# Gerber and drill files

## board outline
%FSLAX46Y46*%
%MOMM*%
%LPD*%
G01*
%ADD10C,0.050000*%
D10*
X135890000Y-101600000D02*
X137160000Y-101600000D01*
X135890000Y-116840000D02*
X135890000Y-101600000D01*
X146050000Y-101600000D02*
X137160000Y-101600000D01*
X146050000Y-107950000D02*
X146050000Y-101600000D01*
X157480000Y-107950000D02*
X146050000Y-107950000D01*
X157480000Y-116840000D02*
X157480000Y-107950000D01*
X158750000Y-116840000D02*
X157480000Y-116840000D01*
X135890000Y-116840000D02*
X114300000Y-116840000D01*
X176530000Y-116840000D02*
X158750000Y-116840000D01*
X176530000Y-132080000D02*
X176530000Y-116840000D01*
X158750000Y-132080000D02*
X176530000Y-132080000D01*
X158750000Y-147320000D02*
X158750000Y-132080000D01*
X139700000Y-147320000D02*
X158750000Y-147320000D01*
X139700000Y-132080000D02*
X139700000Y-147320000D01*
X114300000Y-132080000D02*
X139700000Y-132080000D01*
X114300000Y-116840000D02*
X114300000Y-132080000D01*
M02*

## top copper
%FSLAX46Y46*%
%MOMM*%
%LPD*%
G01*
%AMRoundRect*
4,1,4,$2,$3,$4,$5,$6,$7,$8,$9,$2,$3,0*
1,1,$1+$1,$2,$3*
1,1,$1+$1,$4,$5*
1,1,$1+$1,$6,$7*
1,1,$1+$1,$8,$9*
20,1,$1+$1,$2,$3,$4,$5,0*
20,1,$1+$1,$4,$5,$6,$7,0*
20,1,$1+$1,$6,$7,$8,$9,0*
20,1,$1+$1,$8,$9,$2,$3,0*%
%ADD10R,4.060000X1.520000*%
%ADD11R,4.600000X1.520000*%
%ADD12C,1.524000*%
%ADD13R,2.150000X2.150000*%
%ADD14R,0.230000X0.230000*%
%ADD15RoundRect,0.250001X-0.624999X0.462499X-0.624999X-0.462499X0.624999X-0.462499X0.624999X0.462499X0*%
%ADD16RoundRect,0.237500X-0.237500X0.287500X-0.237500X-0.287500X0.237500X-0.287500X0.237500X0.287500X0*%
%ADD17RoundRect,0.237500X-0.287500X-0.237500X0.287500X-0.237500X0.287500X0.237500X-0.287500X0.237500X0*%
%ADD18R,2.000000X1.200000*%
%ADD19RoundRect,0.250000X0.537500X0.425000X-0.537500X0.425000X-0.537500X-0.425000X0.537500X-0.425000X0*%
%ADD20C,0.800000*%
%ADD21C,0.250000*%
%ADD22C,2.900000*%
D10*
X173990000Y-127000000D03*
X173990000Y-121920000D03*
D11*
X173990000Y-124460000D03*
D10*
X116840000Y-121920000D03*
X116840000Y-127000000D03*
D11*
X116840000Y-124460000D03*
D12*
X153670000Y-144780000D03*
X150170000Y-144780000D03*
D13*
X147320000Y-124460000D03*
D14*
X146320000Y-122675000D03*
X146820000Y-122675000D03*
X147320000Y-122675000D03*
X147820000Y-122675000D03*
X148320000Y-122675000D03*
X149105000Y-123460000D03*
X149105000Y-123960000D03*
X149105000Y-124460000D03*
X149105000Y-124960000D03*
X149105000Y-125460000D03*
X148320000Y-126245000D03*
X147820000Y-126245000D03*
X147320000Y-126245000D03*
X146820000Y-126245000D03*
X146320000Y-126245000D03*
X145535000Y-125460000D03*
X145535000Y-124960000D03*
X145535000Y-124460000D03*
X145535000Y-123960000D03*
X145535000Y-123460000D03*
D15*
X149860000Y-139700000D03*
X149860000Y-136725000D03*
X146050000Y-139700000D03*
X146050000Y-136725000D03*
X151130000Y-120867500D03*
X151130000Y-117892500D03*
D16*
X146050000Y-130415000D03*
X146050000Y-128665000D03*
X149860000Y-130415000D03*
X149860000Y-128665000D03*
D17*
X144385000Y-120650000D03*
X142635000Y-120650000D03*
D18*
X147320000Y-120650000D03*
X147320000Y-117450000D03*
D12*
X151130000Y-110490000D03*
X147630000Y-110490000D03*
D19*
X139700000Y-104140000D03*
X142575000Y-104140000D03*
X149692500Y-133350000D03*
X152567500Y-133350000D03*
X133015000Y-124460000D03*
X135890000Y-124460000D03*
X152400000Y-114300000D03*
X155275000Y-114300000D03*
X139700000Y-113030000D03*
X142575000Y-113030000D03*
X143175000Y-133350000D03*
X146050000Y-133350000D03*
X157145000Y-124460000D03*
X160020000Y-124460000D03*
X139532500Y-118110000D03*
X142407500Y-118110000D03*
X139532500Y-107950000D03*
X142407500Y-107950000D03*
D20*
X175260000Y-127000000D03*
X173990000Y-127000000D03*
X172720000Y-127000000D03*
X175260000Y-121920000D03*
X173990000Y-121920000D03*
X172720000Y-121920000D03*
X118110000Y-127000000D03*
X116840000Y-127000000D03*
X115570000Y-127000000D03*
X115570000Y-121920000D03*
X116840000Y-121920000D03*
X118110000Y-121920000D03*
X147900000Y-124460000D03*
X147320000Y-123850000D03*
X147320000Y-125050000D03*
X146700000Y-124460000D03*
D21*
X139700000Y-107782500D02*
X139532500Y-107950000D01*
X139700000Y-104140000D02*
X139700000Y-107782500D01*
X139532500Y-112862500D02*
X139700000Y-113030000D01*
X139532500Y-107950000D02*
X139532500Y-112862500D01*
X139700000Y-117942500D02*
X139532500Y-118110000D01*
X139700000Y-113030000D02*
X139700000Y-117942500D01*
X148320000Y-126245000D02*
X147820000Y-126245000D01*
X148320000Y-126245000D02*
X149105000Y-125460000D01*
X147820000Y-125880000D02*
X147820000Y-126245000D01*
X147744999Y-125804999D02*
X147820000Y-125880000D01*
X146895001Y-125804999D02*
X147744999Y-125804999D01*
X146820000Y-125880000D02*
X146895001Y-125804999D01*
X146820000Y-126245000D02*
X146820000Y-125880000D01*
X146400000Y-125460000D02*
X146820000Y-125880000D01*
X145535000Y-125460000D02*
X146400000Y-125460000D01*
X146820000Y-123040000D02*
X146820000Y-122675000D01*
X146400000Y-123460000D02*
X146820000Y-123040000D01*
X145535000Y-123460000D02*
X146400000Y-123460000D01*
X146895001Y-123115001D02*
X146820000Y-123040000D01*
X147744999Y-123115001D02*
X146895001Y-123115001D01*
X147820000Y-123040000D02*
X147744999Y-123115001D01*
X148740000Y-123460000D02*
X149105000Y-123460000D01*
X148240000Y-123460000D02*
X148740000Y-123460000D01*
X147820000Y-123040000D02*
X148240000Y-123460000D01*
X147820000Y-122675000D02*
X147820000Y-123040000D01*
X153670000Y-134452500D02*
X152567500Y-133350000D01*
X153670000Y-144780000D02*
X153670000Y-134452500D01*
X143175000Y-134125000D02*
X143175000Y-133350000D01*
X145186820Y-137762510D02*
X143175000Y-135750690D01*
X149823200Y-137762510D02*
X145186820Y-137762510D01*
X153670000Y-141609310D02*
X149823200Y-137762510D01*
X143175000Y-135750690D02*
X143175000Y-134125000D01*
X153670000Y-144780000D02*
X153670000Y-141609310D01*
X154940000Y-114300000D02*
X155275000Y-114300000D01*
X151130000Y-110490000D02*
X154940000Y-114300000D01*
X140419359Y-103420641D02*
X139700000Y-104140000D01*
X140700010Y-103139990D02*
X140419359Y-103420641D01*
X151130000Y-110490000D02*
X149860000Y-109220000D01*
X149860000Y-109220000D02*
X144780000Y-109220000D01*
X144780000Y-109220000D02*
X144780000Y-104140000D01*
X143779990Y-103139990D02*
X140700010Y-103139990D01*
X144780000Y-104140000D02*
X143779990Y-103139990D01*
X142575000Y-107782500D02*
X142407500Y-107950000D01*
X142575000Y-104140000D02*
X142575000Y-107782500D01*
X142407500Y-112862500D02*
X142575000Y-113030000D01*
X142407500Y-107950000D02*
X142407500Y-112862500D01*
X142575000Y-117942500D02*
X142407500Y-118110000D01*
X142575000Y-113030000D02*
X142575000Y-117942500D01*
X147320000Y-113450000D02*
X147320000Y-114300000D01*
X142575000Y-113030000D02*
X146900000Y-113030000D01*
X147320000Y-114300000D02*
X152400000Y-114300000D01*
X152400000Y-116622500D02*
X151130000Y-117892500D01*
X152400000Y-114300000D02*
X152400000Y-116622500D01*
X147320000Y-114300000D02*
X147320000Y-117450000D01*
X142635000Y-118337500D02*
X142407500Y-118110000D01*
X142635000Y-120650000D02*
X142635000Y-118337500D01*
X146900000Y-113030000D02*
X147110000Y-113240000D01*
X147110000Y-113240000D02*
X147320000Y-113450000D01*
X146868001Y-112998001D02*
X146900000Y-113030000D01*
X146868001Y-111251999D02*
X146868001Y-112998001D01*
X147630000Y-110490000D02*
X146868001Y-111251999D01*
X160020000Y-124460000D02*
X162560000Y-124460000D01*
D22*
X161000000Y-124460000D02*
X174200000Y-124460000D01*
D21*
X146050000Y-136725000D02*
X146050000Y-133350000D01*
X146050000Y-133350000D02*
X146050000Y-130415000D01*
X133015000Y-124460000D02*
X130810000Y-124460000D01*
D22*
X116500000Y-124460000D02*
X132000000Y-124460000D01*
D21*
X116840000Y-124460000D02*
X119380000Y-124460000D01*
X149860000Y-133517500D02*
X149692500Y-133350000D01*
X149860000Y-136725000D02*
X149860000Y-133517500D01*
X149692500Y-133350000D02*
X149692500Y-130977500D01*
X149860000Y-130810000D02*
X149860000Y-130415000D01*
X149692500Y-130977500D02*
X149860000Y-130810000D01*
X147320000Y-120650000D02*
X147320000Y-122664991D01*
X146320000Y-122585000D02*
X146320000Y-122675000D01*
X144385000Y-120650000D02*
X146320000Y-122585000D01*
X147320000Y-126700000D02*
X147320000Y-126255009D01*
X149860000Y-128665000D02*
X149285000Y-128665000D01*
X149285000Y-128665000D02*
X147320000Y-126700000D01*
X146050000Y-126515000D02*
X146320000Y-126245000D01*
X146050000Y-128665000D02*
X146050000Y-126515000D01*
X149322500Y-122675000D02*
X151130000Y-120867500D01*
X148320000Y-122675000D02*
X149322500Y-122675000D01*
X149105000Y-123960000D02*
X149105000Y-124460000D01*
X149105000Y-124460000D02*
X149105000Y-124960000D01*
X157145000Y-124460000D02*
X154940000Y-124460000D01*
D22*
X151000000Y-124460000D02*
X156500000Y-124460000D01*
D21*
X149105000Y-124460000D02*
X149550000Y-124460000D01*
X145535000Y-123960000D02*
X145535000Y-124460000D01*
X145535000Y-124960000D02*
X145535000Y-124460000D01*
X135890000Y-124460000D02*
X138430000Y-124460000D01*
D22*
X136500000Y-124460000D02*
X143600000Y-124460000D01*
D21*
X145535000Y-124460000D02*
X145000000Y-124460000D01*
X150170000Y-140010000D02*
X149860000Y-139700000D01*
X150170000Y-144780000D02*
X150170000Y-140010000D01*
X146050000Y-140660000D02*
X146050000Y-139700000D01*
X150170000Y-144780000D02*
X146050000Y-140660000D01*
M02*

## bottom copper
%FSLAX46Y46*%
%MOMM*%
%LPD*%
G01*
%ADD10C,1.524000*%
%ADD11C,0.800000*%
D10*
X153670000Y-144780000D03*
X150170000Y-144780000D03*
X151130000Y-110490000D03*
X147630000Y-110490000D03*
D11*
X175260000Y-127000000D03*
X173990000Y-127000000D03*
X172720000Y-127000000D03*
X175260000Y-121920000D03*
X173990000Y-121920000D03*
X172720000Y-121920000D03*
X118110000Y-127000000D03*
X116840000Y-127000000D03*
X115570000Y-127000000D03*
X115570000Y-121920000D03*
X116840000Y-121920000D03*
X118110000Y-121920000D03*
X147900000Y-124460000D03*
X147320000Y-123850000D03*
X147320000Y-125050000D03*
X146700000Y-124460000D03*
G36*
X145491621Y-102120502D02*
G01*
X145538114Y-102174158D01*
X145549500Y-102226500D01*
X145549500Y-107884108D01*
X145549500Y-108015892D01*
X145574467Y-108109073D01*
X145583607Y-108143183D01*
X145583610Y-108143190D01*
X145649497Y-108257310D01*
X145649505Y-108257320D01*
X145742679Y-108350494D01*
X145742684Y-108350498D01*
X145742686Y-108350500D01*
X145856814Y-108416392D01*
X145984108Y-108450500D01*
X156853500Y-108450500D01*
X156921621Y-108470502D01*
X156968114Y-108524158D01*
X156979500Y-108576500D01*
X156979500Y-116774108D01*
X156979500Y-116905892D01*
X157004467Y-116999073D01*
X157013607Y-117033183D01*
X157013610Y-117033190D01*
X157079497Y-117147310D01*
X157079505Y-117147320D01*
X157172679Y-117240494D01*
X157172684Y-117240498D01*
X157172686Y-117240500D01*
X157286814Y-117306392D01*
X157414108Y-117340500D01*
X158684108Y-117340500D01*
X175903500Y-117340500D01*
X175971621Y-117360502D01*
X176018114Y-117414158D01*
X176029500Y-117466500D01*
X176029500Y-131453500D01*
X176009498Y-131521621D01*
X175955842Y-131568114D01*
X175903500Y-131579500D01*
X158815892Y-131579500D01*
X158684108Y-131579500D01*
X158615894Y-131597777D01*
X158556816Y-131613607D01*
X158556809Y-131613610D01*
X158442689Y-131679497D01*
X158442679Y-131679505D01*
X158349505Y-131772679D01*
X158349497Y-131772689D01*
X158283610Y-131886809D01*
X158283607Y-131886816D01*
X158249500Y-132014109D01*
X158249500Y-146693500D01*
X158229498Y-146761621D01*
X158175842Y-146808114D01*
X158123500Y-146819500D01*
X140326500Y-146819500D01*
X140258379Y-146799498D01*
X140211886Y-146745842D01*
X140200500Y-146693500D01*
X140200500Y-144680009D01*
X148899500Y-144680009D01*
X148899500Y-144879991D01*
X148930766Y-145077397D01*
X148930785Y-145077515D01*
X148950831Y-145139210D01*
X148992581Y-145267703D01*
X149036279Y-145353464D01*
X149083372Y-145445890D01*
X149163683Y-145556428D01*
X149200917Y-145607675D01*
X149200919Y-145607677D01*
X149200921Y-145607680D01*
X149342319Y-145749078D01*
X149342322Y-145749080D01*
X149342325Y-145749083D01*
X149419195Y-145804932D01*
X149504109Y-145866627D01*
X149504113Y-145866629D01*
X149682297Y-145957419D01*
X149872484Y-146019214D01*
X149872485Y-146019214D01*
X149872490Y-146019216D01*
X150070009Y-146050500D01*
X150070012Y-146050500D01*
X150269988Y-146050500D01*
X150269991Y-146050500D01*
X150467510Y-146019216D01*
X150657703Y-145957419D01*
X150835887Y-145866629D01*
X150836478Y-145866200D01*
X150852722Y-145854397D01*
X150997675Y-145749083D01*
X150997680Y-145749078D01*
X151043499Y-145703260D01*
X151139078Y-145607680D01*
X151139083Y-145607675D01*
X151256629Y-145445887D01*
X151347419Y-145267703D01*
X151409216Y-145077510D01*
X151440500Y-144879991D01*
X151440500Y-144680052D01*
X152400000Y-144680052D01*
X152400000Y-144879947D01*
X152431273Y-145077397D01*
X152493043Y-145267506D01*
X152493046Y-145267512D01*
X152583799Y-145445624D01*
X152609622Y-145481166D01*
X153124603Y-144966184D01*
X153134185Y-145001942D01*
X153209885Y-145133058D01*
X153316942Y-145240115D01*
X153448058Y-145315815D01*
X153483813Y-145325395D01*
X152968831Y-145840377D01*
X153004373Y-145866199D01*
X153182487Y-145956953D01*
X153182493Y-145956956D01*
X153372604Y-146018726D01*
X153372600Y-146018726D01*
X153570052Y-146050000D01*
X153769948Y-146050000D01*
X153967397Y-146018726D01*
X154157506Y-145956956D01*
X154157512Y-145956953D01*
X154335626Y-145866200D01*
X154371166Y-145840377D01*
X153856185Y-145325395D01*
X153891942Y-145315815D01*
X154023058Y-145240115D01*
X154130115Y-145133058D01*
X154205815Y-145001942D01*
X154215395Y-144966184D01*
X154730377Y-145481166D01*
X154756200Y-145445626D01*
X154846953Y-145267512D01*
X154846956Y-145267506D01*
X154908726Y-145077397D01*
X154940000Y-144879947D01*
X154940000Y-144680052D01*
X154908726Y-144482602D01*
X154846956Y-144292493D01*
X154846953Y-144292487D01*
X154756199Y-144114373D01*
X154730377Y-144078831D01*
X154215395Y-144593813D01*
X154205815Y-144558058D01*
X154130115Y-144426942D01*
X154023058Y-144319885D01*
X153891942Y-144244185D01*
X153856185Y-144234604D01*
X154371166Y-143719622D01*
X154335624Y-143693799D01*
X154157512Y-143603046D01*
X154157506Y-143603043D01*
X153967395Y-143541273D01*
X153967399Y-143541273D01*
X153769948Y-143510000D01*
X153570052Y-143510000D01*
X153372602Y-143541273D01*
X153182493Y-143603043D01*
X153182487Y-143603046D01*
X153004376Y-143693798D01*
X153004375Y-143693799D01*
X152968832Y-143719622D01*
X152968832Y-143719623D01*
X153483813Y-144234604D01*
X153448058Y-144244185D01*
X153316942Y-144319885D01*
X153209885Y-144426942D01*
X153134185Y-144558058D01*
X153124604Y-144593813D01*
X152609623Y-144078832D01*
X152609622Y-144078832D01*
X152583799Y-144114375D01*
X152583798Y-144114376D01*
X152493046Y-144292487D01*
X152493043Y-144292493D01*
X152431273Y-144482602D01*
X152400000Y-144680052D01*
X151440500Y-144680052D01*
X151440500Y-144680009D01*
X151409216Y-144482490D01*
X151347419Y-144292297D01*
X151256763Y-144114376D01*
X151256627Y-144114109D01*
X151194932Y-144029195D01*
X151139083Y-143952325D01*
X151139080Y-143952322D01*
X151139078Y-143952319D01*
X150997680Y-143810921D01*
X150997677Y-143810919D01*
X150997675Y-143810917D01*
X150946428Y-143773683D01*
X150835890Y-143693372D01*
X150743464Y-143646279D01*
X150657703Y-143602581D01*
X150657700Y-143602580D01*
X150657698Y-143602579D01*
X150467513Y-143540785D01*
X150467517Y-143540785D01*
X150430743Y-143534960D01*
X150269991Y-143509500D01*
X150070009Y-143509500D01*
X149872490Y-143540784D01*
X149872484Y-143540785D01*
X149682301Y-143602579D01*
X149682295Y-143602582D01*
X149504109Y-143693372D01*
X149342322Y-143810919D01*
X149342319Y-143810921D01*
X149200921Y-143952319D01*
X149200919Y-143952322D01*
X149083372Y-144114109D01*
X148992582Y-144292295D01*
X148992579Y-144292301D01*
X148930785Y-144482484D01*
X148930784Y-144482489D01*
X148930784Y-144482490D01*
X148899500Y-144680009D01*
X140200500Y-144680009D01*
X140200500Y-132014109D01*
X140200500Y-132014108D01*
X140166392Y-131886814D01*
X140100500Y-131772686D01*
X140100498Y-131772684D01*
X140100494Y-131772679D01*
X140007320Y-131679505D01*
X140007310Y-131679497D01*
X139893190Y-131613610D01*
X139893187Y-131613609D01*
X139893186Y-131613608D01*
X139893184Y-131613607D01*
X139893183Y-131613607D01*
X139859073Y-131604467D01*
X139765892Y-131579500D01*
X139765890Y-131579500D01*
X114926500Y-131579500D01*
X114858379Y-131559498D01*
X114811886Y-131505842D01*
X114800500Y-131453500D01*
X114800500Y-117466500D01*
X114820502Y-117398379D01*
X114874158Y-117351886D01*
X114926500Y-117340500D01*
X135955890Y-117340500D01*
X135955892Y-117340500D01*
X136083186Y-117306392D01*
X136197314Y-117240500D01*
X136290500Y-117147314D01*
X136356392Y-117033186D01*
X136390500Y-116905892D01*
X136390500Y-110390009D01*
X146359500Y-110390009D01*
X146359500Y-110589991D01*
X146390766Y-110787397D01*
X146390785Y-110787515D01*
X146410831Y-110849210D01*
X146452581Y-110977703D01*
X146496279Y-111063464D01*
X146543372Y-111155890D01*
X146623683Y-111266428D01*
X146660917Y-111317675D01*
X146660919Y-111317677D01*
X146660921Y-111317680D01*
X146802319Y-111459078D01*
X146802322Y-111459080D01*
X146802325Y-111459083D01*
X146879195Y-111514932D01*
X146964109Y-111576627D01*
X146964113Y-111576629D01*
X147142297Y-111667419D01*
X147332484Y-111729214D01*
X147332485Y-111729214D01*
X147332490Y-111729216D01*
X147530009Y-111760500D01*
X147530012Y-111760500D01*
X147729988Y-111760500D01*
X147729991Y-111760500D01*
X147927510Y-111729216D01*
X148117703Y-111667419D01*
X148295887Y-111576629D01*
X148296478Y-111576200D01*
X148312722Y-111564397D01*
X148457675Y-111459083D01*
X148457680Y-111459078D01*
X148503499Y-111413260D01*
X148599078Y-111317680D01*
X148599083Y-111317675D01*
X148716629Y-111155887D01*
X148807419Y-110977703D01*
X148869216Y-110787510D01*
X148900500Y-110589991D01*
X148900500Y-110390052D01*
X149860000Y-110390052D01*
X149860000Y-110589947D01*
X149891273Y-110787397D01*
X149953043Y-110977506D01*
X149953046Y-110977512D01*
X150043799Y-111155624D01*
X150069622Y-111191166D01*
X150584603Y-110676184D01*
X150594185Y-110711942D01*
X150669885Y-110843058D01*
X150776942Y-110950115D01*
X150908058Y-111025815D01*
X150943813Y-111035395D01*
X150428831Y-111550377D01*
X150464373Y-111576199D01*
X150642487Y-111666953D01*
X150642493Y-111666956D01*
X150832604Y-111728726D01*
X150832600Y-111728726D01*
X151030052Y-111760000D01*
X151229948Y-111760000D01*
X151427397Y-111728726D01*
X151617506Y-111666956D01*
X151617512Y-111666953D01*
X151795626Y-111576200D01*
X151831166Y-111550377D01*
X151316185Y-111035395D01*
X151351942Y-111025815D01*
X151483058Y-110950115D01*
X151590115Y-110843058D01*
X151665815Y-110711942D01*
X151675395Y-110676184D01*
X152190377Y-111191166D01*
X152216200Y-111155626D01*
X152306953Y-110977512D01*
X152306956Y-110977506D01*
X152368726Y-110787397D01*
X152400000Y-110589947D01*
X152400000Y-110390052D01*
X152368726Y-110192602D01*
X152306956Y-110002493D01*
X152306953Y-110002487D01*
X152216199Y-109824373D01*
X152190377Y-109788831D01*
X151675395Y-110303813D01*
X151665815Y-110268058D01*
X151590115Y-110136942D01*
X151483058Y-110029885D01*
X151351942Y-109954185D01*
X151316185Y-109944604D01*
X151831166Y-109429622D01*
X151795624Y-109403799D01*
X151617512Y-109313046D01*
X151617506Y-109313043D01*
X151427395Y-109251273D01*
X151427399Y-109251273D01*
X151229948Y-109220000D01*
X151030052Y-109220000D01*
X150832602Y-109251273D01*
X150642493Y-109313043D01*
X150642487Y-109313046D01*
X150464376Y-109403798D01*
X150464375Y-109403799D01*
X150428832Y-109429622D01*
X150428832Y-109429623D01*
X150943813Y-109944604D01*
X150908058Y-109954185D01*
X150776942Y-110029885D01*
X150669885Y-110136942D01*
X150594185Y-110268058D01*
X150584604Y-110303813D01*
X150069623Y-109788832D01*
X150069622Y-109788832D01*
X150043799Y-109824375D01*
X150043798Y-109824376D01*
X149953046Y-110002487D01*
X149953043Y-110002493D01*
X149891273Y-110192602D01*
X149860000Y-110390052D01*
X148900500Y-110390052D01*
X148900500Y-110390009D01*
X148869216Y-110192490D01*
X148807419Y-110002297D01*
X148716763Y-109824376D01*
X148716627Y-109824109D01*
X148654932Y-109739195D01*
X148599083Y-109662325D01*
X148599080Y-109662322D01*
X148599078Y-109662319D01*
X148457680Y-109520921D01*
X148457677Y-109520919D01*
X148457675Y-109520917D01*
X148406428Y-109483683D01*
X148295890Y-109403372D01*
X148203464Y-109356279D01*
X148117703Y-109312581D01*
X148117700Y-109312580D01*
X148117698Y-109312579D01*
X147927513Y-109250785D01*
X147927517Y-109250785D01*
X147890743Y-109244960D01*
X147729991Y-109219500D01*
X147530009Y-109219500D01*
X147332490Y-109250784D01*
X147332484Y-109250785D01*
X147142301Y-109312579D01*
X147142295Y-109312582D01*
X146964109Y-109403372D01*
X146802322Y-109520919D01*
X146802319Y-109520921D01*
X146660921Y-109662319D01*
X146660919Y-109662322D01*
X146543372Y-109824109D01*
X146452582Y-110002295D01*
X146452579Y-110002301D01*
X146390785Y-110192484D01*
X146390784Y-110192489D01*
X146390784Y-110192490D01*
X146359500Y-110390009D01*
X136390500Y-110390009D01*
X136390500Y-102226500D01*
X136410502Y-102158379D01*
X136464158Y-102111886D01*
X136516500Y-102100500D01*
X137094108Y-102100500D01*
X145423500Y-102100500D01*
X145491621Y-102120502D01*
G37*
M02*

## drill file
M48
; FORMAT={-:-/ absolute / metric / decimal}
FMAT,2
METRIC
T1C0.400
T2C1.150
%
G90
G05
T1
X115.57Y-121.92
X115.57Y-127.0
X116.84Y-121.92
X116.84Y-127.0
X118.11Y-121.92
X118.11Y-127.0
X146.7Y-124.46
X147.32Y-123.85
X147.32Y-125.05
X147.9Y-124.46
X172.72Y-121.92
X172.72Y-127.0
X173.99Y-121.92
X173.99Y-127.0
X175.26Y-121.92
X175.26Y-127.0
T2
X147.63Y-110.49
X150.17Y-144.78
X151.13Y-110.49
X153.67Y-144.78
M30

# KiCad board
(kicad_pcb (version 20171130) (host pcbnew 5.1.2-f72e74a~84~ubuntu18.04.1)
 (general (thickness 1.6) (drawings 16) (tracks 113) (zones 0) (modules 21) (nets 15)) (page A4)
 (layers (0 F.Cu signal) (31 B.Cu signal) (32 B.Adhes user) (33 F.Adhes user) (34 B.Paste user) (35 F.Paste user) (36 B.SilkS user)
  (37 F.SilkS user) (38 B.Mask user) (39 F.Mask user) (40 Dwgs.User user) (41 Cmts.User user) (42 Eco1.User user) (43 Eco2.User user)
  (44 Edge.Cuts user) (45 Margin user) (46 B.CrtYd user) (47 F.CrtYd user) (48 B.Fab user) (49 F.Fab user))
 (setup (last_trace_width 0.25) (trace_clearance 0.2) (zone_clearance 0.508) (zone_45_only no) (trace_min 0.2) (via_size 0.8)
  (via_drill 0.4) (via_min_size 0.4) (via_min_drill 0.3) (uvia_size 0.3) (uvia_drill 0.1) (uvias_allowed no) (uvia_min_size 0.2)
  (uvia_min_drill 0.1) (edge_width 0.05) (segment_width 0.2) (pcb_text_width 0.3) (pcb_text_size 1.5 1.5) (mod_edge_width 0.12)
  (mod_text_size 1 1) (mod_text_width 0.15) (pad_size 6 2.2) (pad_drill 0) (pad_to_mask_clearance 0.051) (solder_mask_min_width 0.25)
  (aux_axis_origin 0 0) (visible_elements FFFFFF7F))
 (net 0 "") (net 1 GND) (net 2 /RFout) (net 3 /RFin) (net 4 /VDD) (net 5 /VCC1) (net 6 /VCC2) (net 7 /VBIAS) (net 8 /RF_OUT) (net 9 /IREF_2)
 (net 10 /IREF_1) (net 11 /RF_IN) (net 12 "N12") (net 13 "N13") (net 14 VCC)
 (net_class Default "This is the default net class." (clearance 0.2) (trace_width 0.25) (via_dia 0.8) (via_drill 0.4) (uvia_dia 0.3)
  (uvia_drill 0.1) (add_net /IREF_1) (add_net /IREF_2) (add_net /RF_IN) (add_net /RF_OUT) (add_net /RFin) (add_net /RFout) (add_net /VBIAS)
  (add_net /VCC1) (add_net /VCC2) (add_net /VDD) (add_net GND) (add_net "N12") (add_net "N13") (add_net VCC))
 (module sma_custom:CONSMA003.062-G (layer F.Cu) (at 177.8 127)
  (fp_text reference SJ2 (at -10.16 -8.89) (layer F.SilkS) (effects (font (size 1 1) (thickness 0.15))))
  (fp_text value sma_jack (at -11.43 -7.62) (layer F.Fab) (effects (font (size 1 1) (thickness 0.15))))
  (pad 3 smd rect (at -3.81 0) (size 4.06 1.52) (layers F.Cu F.Paste F.Mask) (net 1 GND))
  (pad 2 smd rect (at -3.81 -5.08) (size 4.06 1.52) (layers F.Cu F.Paste F.Mask) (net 1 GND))
  (pad 1 smd rect (at -3.81 -2.54) (size 4.6 1.52) (layers F.Cu F.Paste F.Mask) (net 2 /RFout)))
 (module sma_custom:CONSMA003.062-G (layer F.Cu) (at 113.03 121.92 180)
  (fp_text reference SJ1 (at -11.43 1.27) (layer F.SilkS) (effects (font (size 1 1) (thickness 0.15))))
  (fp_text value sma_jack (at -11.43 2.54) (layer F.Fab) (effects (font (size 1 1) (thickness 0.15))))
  (pad 3 smd rect (at -3.81 0 180) (size 4.06 1.52) (layers F.Cu F.Paste F.Mask) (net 1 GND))
  (pad 2 smd rect (at -3.81 -5.08 180) (size 4.06 1.52) (layers F.Cu F.Paste F.Mask) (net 1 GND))
  (pad 1 smd rect (at -3.81 -2.54 180) (size 4.6 1.52) (layers F.Cu F.Paste F.Mask) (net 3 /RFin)))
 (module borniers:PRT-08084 (layer F.Cu) (at 153.67 149.86)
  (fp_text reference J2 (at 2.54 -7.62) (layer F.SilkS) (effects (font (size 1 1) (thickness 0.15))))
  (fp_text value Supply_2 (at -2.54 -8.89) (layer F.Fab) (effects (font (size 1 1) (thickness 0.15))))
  (pad 2 thru_hole circle (at 0 -5.08) (size 1.524 1.524) (drill 1.15) (layers *.Cu *.Mask) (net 1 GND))
  (pad 1 thru_hole circle (at -3.5 -5.08) (size 1.524 1.524) (drill 1.15) (layers *.Cu *.Mask) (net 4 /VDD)))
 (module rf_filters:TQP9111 (layer F.Cu) (at 147.32 124.46)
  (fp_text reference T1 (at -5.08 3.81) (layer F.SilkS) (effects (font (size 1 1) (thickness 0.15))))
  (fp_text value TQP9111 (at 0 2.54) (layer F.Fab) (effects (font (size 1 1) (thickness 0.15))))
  (pad 21 smd rect (at 0 0) (size 2.15 2.15) (layers F.Cu F.Paste F.Mask) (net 1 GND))
  (pad 20 smd rect (at -1 -1.785) (size 0.23 0.23) (layers F.Cu F.Paste F.Mask) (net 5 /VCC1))
  (pad 19 smd rect (at -0.5 -1.785) (size 0.23 0.23) (layers F.Cu F.Paste F.Mask) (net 1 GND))
  (pad 18 smd rect (at 0 -1.785) (size 0.23 0.23) (layers F.Cu F.Paste F.Mask) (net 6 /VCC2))
  (pad 17 smd rect (at 0.5 -1.785) (size 0.23 0.23) (layers F.Cu F.Paste F.Mask) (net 1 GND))
  (pad 16 smd rect (at 1 -1.785) (size 0.23 0.23) (layers F.Cu F.Paste F.Mask) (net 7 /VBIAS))
  (pad 15 smd rect (at 1.785 -1) (size 0.23 0.23) (layers F.Cu F.Paste F.Mask) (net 1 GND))
  (pad 14 smd rect (at 1.785 -0.5) (size 0.23 0.23) (layers F.Cu F.Paste F.Mask) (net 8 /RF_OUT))
  (pad 13 smd rect (at 1.785 0) (size 0.23 0.23) (layers F.Cu F.Paste F.Mask) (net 8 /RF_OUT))
  (pad 12 smd rect (at 1.785 0.5) (size 0.23 0.23) (layers F.Cu F.Paste F.Mask) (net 8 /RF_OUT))
  (pad 11 smd rect (at 1.785 1) (size 0.23 0.23) (layers F.Cu F.Paste F.Mask) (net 1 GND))
  (pad 10 smd rect (at 1 1.785) (size 0.23 0.23) (layers F.Cu F.Paste F.Mask) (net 1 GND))
  (pad 9 smd rect (at 0.5 1.785) (size 0.23 0.23) (layers F.Cu F.Paste F.Mask) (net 1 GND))
  (pad 8 smd rect (at 0 1.785) (size 0.23 0.23) (layers F.Cu F.Paste F.Mask) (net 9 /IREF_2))
  (pad 7 smd rect (at -0.5 1.785) (size 0.23 0.23) (layers F.Cu F.Paste F.Mask) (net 1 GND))
  (pad 6 smd rect (at -1 1.785) (size 0.23 0.23) (layers F.Cu F.Paste F.Mask) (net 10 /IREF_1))
  (pad 5 smd rect (at -1.785 1) (size 0.23 0.23) (layers F.Cu F.Paste F.Mask) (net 1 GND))
  (pad 4 smd rect (at -1.785 0.5) (size 0.23 0.23) (layers F.Cu F.Paste F.Mask) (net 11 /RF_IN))
  (pad 3 smd rect (at -1.785 0) (size 0.23 0.23) (layers F.Cu F.Paste F.Mask) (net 11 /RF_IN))
  (pad 2 smd rect (at -1.785 -0.5) (size 0.23 0.23) (layers F.Cu F.Paste F.Mask) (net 11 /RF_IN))
  (pad 1 smd rect (at -1.785 -1) (size 0.23 0.23) (layers F.Cu F.Paste F.Mask) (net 1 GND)))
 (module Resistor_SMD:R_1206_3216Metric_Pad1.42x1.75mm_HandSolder (layer F.Cu) (at 149.86 138.2125 270)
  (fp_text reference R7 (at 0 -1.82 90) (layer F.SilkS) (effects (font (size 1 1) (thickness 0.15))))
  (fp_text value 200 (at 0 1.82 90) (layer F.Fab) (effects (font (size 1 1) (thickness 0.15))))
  (pad 2 smd roundrect (at 1.4875 0 270) (size 1.425 1.75) (layers F.Cu F.Paste F.Mask) (roundrect_rratio 0.175439) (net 4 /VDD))
  (pad 1 smd roundrect (at -1.4875 0 270) (size 1.425 1.75) (layers F.Cu F.Paste F.Mask) (roundrect_rratio 0.175439) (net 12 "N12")))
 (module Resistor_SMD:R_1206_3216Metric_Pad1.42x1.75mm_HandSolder (layer F.Cu) (at 146.05 138.2125 270)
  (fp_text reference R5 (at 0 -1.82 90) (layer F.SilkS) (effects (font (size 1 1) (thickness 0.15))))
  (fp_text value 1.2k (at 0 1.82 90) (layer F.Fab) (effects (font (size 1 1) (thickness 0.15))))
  (pad 2 smd roundrect (at 1.4875 0 270) (size 1.425 1.75) (layers F.Cu F.Paste F.Mask) (roundrect_rratio 0.175439) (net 4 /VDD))
  (pad 1 smd roundrect (at -1.4875 0 270) (size 1.425 1.75) (layers F.Cu F.Paste F.Mask) (roundrect_rratio 0.175439) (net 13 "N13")))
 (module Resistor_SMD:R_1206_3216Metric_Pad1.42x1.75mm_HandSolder (layer F.Cu) (at 151.13 119.38 270)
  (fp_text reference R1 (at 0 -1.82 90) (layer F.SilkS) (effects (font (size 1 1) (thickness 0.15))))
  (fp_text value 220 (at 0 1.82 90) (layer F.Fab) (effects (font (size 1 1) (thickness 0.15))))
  (pad 2 smd roundrect (at 1.4875 0 270) (size 1.425 1.75) (layers F.Cu F.Paste F.Mask) (roundrect_rratio 0.175439) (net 7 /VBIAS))
  (pad 1 smd roundrect (at -1.4875 0 270) (size 1.425 1.75) (layers F.Cu F.Paste F.Mask) (roundrect_rratio 0.175439) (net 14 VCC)))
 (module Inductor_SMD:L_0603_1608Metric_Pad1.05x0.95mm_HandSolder (layer F.Cu) (at 146.05 129.54 270)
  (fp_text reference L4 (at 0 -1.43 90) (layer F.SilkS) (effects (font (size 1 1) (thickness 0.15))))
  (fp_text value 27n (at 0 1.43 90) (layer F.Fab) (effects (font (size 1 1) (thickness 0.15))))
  (pad 2 smd roundrect (at 0.875 0 270) (size 1.05 0.95) (layers F.Cu F.Paste F.Mask) (roundrect_rratio 0.25) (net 13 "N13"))
  (pad 1 smd roundrect (at -0.875 0 270) (size 1.05 0.95) (layers F.Cu F.Paste F.Mask) (roundrect_rratio 0.25) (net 10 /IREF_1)))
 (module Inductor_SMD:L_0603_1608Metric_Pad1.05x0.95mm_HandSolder (layer F.Cu) (at 149.86 129.54 270)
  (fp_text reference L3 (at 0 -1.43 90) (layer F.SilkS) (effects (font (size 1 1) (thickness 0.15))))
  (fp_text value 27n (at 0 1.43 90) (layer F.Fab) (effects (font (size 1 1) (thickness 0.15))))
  (pad 2 smd roundrect (at 0.875 0 270) (size 1.05 0.95) (layers F.Cu F.Paste F.Mask) (roundrect_rratio 0.25) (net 12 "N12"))
  (pad 1 smd roundrect (at -0.875 0 270) (size 1.05 0.95) (layers F.Cu F.Paste F.Mask) (roundrect_rratio 0.25) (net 9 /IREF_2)))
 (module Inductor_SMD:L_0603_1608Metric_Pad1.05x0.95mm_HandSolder (layer F.Cu) (at 143.51 120.65)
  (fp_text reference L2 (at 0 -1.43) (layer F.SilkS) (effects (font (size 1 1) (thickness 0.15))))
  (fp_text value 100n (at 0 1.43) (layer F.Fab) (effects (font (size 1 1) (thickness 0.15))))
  (pad 2 smd roundrect (at 0.875 0) (size 1.05 0.95) (layers F.Cu F.Paste F.Mask) (roundrect_rratio 0.25) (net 5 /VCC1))
  (pad 1 smd roundrect (at -0.875 0) (size 1.05 0.95) (layers F.Cu F.Paste F.Mask) (roundrect_rratio 0.25) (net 14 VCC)))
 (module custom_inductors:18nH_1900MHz (layer F.Cu) (at 147.32 119.05)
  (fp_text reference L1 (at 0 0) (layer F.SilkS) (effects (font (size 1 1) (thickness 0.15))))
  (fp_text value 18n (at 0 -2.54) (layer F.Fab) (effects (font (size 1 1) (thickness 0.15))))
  (pad 2 smd rect (at 0 1.6) (size 2 1.2) (layers F.Cu F.Paste F.Mask) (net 6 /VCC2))
  (pad 1 smd rect (at 0 -1.6) (size 2 1.2) (layers F.Cu F.Paste F.Mask) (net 14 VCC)))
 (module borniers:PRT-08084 (layer F.Cu) (at 151.13 115.57)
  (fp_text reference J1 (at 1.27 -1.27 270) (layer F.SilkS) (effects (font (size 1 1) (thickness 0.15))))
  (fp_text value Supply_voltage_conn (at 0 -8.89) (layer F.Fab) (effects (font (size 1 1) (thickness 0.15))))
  (pad 2 thru_hole circle (at 0 -5.08) (size 1.524 1.524) (drill 1.15) (layers *.Cu *.Mask) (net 1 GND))
  (pad 1 thru_hole circle (at -3.5 -5.08) (size 1.524 1.524) (drill 1.15) (layers *.Cu *.Mask) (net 14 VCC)))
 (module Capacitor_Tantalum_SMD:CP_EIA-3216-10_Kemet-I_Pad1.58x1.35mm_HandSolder (layer F.Cu) (at 141.1375 104.14 180)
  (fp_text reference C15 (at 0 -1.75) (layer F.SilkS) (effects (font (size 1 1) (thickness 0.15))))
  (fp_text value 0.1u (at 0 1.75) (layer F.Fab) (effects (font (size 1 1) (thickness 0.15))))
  (pad 2 smd roundrect (at 1.4375 0 180) (size 1.575 1.35) (layers F.Cu F.Paste F.Mask) (roundrect_rratio 0.185185) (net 1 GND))
  (pad 1 smd roundrect (at -1.4375 0 180) (size 1.575 1.35) (layers F.Cu F.Paste F.Mask) (roundrect_rratio 0.185185) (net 14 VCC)))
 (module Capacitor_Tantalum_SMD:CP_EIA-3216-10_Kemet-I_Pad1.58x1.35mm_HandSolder (layer F.Cu) (at 151.13 133.35 180)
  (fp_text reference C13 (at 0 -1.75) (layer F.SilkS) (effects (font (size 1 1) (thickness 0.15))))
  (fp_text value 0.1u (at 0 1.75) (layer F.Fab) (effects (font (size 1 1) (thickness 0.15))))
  (pad 2 smd roundrect (at 1.4375 0 180) (size 1.575 1.35) (layers F.Cu F.Paste F.Mask) (roundrect_rratio 0.185185) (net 12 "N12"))
  (pad 1 smd roundrect (at -1.4375 0 180) (size 1.575 1.35) (layers F.Cu F.Paste F.Mask) (roundrect_rratio 0.185185) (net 1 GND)))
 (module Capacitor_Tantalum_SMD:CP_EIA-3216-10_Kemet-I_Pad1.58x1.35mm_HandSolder (layer F.Cu) (at 134.4525 124.46 180)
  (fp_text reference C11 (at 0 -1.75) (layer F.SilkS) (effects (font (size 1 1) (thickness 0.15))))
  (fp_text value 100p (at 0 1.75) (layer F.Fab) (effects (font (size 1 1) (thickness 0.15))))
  (pad 2 smd roundrect (at 1.4375 0 180) (size 1.575 1.35) (layers F.Cu F.Paste F.Mask) (roundrect_rratio 0.185185) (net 3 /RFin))
  (pad 1 smd roundrect (at -1.4375 0 180) (size 1.575 1.35) (layers F.Cu F.Paste F.Mask) (roundrect_rratio 0.185185) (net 11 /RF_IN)))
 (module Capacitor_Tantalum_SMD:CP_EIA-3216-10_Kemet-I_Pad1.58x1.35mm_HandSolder (layer F.Cu) (at 153.8375 114.3 180)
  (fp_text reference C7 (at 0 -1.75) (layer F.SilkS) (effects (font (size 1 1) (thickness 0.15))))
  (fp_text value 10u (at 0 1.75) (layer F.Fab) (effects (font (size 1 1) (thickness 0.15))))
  (pad 2 smd roundrect (at 1.4375 0 180) (size 1.575 1.35) (layers F.Cu F.Paste F.Mask) (roundrect_rratio 0.185185) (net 14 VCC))
  (pad 1 smd roundrect (at -1.4375 0 180) (size 1.575 1.35) (layers F.Cu F.Paste F.Mask) (roundrect_rratio 0.185185) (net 1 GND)))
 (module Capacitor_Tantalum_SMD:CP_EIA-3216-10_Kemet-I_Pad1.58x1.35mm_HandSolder (layer F.Cu) (at 141.1375 113.03 180)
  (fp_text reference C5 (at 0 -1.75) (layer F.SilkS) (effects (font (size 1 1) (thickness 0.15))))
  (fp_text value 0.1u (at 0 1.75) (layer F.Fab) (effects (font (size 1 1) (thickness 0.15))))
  (pad 2 smd roundrect (at 1.4375 0 180) (size 1.575 1.35) (layers F.Cu F.Paste F.Mask) (roundrect_rratio 0.185185) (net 1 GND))
  (pad 1 smd roundrect (at -1.4375 0 180) (size 1.575 1.35) (layers F.Cu F.Paste F.Mask) (roundrect_rratio 0.185185) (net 14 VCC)))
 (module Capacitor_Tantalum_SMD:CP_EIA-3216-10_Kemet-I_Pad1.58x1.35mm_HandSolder (layer F.Cu) (at 144.6125 133.35 180)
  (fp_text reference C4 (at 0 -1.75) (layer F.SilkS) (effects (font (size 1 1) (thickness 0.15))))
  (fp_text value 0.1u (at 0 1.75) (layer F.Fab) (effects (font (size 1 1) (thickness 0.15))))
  (pad 2 smd roundrect (at 1.4375 0 180) (size 1.575 1.35) (layers F.Cu F.Paste F.Mask) (roundrect_rratio 0.185185) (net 1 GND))
  (pad 1 smd roundrect (at -1.4375 0 180) (size 1.575 1.35) (layers F.Cu F.Paste F.Mask) (roundrect_rratio 0.185185) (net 13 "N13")))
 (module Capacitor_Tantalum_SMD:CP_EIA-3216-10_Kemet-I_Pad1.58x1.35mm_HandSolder (layer F.Cu) (at 158.5825 124.46 180)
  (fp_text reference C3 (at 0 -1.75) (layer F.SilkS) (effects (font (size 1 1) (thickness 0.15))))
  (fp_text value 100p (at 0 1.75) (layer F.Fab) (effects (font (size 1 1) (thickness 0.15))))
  (pad 2 smd roundrect (at 1.4375 0 180) (size 1.575 1.35) (layers F.Cu F.Paste F.Mask) (roundrect_rratio 0.185185) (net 8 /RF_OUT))
  (pad 1 smd roundrect (at -1.4375 0 180) (size 1.575 1.35) (layers F.Cu F.Paste F.Mask) (roundrect_rratio 0.185185) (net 2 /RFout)))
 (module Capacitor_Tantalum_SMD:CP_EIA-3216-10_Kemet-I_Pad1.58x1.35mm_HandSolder (layer F.Cu) (at 140.97 118.11 180)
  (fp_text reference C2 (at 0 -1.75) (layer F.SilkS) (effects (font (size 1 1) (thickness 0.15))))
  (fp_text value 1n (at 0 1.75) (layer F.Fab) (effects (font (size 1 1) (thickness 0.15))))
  (pad 2 smd roundrect (at 1.4375 0 180) (size 1.575 1.35) (layers F.Cu F.Paste F.Mask) (roundrect_rratio 0.185185) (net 1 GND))
  (pad 1 smd roundrect (at -1.4375 0 180) (size 1.575 1.35) (layers F.Cu F.Paste F.Mask) (roundrect_rratio 0.185185) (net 14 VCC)))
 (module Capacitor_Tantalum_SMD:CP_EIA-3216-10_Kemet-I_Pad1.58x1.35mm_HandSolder (layer F.Cu) (at 140.97 107.95 180)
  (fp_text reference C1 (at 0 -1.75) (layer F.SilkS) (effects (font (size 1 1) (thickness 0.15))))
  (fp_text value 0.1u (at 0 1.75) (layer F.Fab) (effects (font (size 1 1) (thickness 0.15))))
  (pad 2 smd roundrect (at 1.4375 0 180) (size 1.575 1.35) (layers F.Cu F.Paste F.Mask) (roundrect_rratio 0.185185) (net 1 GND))
  (pad 1 smd roundrect (at -1.4375 0 180) (size 1.575 1.35) (layers F.Cu F.Paste F.Mask) (roundrect_rratio 0.185185) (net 14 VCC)))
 (gr_line (start 135.89 101.6) (end 137.16 101.6) (layer Edge.Cuts) (width 0.05))
 (gr_line (start 135.89 116.84) (end 135.89 101.6) (layer Edge.Cuts) (width 0.05))
 (gr_line (start 146.05 101.6) (end 137.16 101.6) (layer Edge.Cuts) (width 0.05))
 (gr_line (start 146.05 107.95) (end 146.05 101.6) (layer Edge.Cuts) (width 0.05))
 (gr_line (start 157.48 107.95) (end 146.05 107.95) (layer Edge.Cuts) (width 0.05))
 (gr_line (start 157.48 116.84) (end 157.48 107.95) (layer Edge.Cuts) (width 0.05))
 (gr_line (start 158.75 116.84) (end 157.48 116.84) (layer Edge.Cuts) (width 0.05))
 (gr_line (start 135.89 116.84) (end 114.3 116.84) (layer Edge.Cuts) (width 0.05))
 (gr_line (start 176.53 116.84) (end 158.75 116.84) (layer Edge.Cuts) (width 0.05))
 (gr_line (start 176.53 132.08) (end 176.53 116.84) (layer Edge.Cuts) (width 0.05))
 (gr_line (start 158.75 132.08) (end 176.53 132.08) (layer Edge.Cuts) (width 0.05))
 (gr_line (start 158.75 147.32) (end 158.75 132.08) (layer Edge.Cuts) (width 0.05))
 (gr_line (start 139.7 147.32) (end 158.75 147.32) (layer Edge.Cuts) (width 0.05))
 (gr_line (start 139.7 132.08) (end 139.7 147.32) (layer Edge.Cuts) (width 0.05))
 (gr_line (start 114.3 132.08) (end 139.7 132.08) (layer Edge.Cuts) (width 0.05))
 (gr_line (start 114.3 116.84) (end 114.3 132.08) (layer Edge.Cuts) (width 0.05))
 (via (at 175.26 127) (size 0.8) (drill 0.4) (layers F.Cu B.Cu) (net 1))
 (via (at 173.99 127) (size 0.8) (drill 0.4) (layers F.Cu B.Cu) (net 1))
 (via (at 172.72 127) (size 0.8) (drill 0.4) (layers F.Cu B.Cu) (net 1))
 (via (at 175.26 121.92) (size 0.8) (drill 0.4) (layers F.Cu B.Cu) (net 1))
 (via (at 173.99 121.92) (size 0.8) (drill 0.4) (layers F.Cu B.Cu) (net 1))
 (via (at 172.72 121.92) (size 0.8) (drill 0.4) (layers F.Cu B.Cu) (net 1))
 (via (at 118.11 127) (size 0.8) (drill 0.4) (layers F.Cu B.Cu) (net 1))
 (via (at 116.84 127) (size 0.8) (drill 0.4) (layers F.Cu B.Cu) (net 1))
 (via (at 115.57 127) (size 0.8) (drill 0.4) (layers F.Cu B.Cu) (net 1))
 (via (at 115.57 121.92) (size 0.8) (drill 0.4) (layers F.Cu B.Cu) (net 1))
 (via (at 116.84 121.92) (size 0.8) (drill 0.4) (layers F.Cu B.Cu) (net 1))
 (via (at 118.11 121.92) (size 0.8) (drill 0.4) (layers F.Cu B.Cu) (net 1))
 (via (at 147.9 124.46) (size 0.8) (drill 0.4) (layers F.Cu B.Cu) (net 1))
 (via (at 147.32 123.85) (size 0.8) (drill 0.4) (layers F.Cu B.Cu) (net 1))
 (segment (start 139.7 107.7825) (end 139.5325 107.95) (width 0.25) (layer F.Cu) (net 1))
 (segment (start 139.7 104.14) (end 139.7 107.7825) (width 0.25) (layer F.Cu) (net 1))
 (segment (start 139.5325 112.8625) (end 139.7 113.03) (width 0.25) (layer F.Cu) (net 1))
 (segment (start 139.5325 107.95) (end 139.5325 112.8625) (width 0.25) (layer F.Cu) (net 1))
 (segment (start 139.7 117.9425) (end 139.5325 118.11) (width 0.25) (layer F.Cu) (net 1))
 (segment (start 139.7 113.03) (end 139.7 117.9425) (width 0.25) (layer F.Cu) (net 1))
 (via (at 147.32 125.05) (size 0.8) (drill 0.4) (layers F.Cu B.Cu) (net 1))
 (via (at 146.7 124.46) (size 0.8) (drill 0.4) (layers F.Cu B.Cu) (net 1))
 (segment (start 148.32 126.245) (end 147.82 126.245) (width 0.25) (layer F.Cu) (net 1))
 (segment (start 148.32 126.245) (end 149.105 125.46) (width 0.25) (layer F.Cu) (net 1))
 (segment (start 147.82 125.88) (end 147.82 126.245) (width 0.25) (layer F.Cu) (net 1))
 (segment (start 147.744999 125.804999) (end 147.82 125.88) (width 0.25) (layer F.Cu) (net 1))
 (segment (start 146.895001 125.804999) (end 147.744999 125.804999) (width 0.25) (layer F.Cu) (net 1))
 (segment (start 146.82 125.88) (end 146.895001 125.804999) (width 0.25) (layer F.Cu) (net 1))
 (segment (start 146.82 126.245) (end 146.82 125.88) (width 0.25) (layer F.Cu) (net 1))
 (segment (start 146.4 125.46) (end 146.82 125.88) (width 0.25) (layer F.Cu) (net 1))
 (segment (start 145.535 125.46) (end 146.4 125.46) (width 0.25) (layer F.Cu) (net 1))
 (segment (start 146.82 123.04) (end 146.82 122.675) (width 0.25) (layer F.Cu) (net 1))
 (segment (start 146.4 123.46) (end 146.82 123.04) (width 0.25) (layer F.Cu) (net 1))
 (segment (start 145.535 123.46) (end 146.4 123.46) (width 0.25) (layer F.Cu) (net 1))
 (segment (start 146.895001 123.115001) (end 146.82 123.04) (width 0.25) (layer F.Cu) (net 1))
 (segment (start 147.744999 123.115001) (end 146.895001 123.115001) (width 0.25) (layer F.Cu) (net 1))
 (segment (start 147.82 123.04) (end 147.744999 123.115001) (width 0.25) (layer F.Cu) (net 1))
 (segment (start 148.74 123.46) (end 149.105 123.46) (width 0.25) (layer F.Cu) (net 1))
 (segment (start 148.24 123.46) (end 148.74 123.46) (width 0.25) (layer F.Cu) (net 1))
 (segment (start 147.82 123.04) (end 148.24 123.46) (width 0.25) (layer F.Cu) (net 1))
 (segment (start 147.82 122.675) (end 147.82 123.04) (width 0.25) (layer F.Cu) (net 1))
 (segment (start 153.67 134.4525) (end 152.5675 133.35) (width 0.25) (layer F.Cu) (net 1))
 (segment (start 153.67 144.78) (end 153.67 134.4525) (width 0.25) (layer F.Cu) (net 1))
 (segment (start 143.175 134.125) (end 143.175 133.35) (width 0.25) (layer F.Cu) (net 1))
 (segment (start 145.18682 137.76251) (end 143.175 135.75069) (width 0.25) (layer F.Cu) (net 1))
 (segment (start 149.8232 137.76251) (end 145.18682 137.76251) (width 0.25) (layer F.Cu) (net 1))
 (segment (start 153.67 141.60931) (end 149.8232 137.76251) (width 0.25) (layer F.Cu) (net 1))
 (segment (start 143.175 135.75069) (end 143.175 134.125) (width 0.25) (layer F.Cu) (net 1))
 (segment (start 153.67 144.78) (end 153.67 141.60931) (width 0.25) (layer F.Cu) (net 1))
 (segment (start 154.94 114.3) (end 155.275 114.3) (width 0.25) (layer F.Cu) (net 1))
 (segment (start 151.13 110.49) (end 154.94 114.3) (width 0.25) (layer F.Cu) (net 1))
 (segment (start 140.419359 103.420641) (end 139.7 104.14) (width 0.25) (layer F.Cu) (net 1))
 (segment (start 140.70001 103.13999) (end 140.419359 103.420641) (width 0.25) (layer F.Cu) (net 1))
 (segment (start 151.13 110.49) (end 149.86 109.22) (width 0.25) (layer F.Cu) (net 1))
 (segment (start 149.86 109.22) (end 144.78 109.22) (width 0.25) (layer F.Cu) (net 1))
 (segment (start 144.78 109.22) (end 144.78 104.14) (width 0.25) (layer F.Cu) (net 1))
 (segment (start 143.77999 103.13999) (end 140.70001 103.13999) (width 0.25) (layer F.Cu) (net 1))
 (segment (start 144.78 104.14) (end 143.77999 103.13999) (width 0.25) (layer F.Cu) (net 1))
 (segment (start 142.575 107.7825) (end 142.4075 107.95) (width 0.25) (layer F.Cu) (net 14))
 (segment (start 142.575 104.14) (end 142.575 107.7825) (width 0.25) (layer F.Cu) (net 14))
 (segment (start 142.4075 112.8625) (end 142.575 113.03) (width 0.25) (layer F.Cu) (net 14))
 (segment (start 142.4075 107.95) (end 142.4075 112.8625) (width 0.25) (layer F.Cu) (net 14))
 (segment (start 142.575 117.9425) (end 142.4075 118.11) (width 0.25) (layer F.Cu) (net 14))
 (segment (start 142.575 113.03) (end 142.575 117.9425) (width 0.25) (layer F.Cu) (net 14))
 (segment (start 147.32 113.45) (end 147.32 114.3) (width 0.25) (layer F.Cu) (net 14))
 (segment (start 142.575 113.03) (end 146.9 113.03) (width 0.25) (layer F.Cu) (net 14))
 (segment (start 147.32 114.3) (end 152.4 114.3) (width 0.25) (layer F.Cu) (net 14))
 (segment (start 152.4 116.6225) (end 151.13 117.8925) (width 0.25) (layer F.Cu) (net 14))
 (segment (start 152.4 114.3) (end 152.4 116.6225) (width 0.25) (layer F.Cu) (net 14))
 (segment (start 147.32 114.3) (end 147.32 117.45) (width 0.25) (layer F.Cu) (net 14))
 (segment (start 142.635 118.3375) (end 142.4075 118.11) (width 0.25) (layer F.Cu) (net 14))
 (segment (start 142.635 120.65) (end 142.635 118.3375) (width 0.25) (layer F.Cu) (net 14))
 (segment (start 146.9 113.03) (end 147.11 113.24) (width 0.25) (layer F.Cu) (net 14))
 (segment (start 147.11 113.24) (end 147.32 113.45) (width 0.25) (layer F.Cu) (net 14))
 (segment (start 146.868001 112.998001) (end 146.9 113.03) (width 0.25) (layer F.Cu) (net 14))
 (segment (start 146.868001 111.251999) (end 146.868001 112.998001) (width 0.25) (layer F.Cu) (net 14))
 (segment (start 147.63 110.49) (end 146.868001 111.251999) (width 0.25) (layer F.Cu) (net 14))
 (segment (start 160.02 124.46) (end 162.56 124.46) (width 0.25) (layer F.Cu) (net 2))
 (segment (start 161 124.46) (end 174.2 124.46) (width 2.9) (layer F.Cu) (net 2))
 (segment (start 146.05 136.725) (end 146.05 133.35) (width 0.25) (layer F.Cu) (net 13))
 (segment (start 146.05 133.35) (end 146.05 130.415) (width 0.25) (layer F.Cu) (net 13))
 (segment (start 133.015 124.46) (end 130.81 124.46) (width 0.25) (layer F.Cu) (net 3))
 (segment (start 116.5 124.46) (end 132 124.46) (width 2.9) (layer F.Cu) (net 3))
 (segment (start 116.84 124.46) (end 119.38 124.46) (width 0.25) (layer F.Cu) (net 3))
 (segment (start 149.86 133.5175) (end 149.6925 133.35) (width 0.25) (layer F.Cu) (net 12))
 (segment (start 149.86 136.725) (end 149.86 133.5175) (width 0.25) (layer F.Cu) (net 12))
 (segment (start 149.6925 133.35) (end 149.6925 130.9775) (width 0.25) (layer F.Cu) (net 12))
 (segment (start 149.86 130.81) (end 149.86 130.415) (width 0.25) (layer F.Cu) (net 12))
 (segment (start 149.6925 130.9775) (end 149.86 130.81) (width 0.25) (layer F.Cu) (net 12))
 (segment (start 147.32 120.65) (end 147.32 122.664991) (width 0.25) (layer F.Cu) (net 6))
 (segment (start 146.32 122.585) (end 146.32 122.675) (width 0.25) (layer F.Cu) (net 5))
 (segment (start 144.385 120.65) (end 146.32 122.585) (width 0.25) (layer F.Cu) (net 5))
 (segment (start 147.32 126.7) (end 147.32 126.255009) (width 0.25) (layer F.Cu) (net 9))
 (segment (start 149.86 128.665) (end 149.285 128.665) (width 0.25) (layer F.Cu) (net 9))
 (segment (start 149.285 128.665) (end 147.32 126.7) (width 0.25) (layer F.Cu) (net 9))
 (segment (start 146.05 126.515) (end 146.32 126.245) (width 0.25) (layer F.Cu) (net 10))
 (segment (start 146.05 128.665) (end 146.05 126.515) (width 0.25) (layer F.Cu) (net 10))
 (segment (start 149.3225 122.675) (end 151.13 120.8675) (width 0.25) (layer F.Cu) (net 7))
 (segment (start 148.32 122.675) (end 149.3225 122.675) (width 0.25) (layer F.Cu) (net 7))
 (segment (start 149.105 123.96) (end 149.105 124.46) (width 0.25) (layer F.Cu) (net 8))
 (segment (start 149.105 124.46) (end 149.105 124.96) (width 0.25) (layer F.Cu) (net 8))
 (segment (start 157.145 124.46) (end 154.94 124.46) (width 0.25) (layer F.Cu) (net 8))
 (segment (start 151 124.46) (end 156.5 124.46) (width 2.9) (layer F.Cu) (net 8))
 (segment (start 149.105 124.46) (end 149.55 124.46) (width 0.25) (layer F.Cu) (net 8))
 (segment (start 145.535 123.96) (end 145.535 124.46) (width 0.25) (layer F.Cu) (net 11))
 (segment (start 145.535 124.96) (end 145.535 124.46) (width 0.25) (layer F.Cu) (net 11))
 (segment (start 135.89 124.46) (end 138.43 124.46) (width 0.25) (layer F.Cu) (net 11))
 (segment (start 136.5 124.46) (end 143.6 124.46) (width 2.9) (layer F.Cu) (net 11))
 (segment (start 145.535 124.46) (end 145 124.46) (width 0.25) (layer F.Cu) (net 11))
 (segment (start 150.17 140.01) (end 149.86 139.7) (width 0.25) (layer F.Cu) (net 4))
 (segment (start 150.17 144.78) (end 150.17 140.01) (width 0.25) (layer F.Cu) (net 4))
 (segment (start 146.05 140.66) (end 146.05 139.7) (width 0.25) (layer F.Cu) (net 4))
 (segment (start 150.17 144.78) (end 146.05 140.66) (width 0.25) (layer F.Cu) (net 4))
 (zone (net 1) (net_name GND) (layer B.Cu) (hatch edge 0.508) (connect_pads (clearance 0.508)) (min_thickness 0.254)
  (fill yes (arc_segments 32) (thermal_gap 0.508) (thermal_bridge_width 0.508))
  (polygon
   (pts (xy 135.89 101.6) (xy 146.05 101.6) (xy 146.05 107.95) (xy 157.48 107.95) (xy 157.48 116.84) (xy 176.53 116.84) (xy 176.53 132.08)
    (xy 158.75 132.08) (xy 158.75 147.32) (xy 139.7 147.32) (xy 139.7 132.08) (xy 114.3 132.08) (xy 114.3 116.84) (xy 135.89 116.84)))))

